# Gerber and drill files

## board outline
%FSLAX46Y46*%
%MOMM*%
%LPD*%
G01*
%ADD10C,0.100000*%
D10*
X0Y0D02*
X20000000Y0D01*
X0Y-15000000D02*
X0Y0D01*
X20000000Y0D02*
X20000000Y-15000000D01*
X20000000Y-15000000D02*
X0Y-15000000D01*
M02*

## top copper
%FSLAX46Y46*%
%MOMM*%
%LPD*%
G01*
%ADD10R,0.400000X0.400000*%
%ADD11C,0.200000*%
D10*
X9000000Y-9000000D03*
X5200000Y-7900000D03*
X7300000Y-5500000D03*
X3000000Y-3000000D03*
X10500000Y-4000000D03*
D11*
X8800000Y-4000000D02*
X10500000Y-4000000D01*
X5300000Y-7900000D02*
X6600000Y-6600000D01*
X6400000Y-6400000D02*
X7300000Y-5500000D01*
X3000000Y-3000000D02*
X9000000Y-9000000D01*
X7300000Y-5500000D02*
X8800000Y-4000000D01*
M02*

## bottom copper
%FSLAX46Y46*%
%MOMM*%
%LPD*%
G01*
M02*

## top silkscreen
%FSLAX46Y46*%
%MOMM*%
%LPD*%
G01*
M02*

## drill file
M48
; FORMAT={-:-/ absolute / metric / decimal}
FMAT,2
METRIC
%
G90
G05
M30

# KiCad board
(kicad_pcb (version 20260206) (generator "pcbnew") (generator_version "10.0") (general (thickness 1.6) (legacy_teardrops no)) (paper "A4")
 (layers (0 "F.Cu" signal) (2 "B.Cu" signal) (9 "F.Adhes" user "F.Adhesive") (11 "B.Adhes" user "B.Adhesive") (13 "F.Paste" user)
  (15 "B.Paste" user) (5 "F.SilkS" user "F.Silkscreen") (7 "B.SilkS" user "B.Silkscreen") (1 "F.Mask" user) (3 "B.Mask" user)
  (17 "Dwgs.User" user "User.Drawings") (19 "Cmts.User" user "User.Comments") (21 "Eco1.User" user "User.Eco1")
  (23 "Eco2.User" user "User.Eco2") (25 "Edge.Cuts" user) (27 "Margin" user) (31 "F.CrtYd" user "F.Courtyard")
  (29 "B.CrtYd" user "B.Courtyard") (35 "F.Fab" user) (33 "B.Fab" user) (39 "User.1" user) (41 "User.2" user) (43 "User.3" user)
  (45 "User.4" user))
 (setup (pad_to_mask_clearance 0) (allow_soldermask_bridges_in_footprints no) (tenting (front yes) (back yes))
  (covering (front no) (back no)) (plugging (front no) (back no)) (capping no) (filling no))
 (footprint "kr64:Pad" (layer "F.Cu") (at 9 9)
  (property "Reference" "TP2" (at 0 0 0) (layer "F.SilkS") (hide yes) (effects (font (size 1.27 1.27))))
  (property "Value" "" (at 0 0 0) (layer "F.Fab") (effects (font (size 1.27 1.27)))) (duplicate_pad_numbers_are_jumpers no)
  (pad "1" smd rect (at 0 0) (size 0.4 0.4) (layers "F.Cu" "F.Mask" "F.Paste") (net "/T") (thermal_bridge_angle 45)))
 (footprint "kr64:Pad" (layer "F.Cu") (at 5.2 7.9)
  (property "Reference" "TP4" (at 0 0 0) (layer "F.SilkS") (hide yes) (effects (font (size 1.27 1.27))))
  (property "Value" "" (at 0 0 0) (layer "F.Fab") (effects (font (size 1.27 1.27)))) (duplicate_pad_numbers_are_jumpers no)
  (pad "1" smd rect (at 0 0) (size 0.4 0.4) (layers "F.Cu" "F.Mask" "F.Paste") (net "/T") (thermal_bridge_angle 45)))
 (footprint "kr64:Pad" (layer "F.Cu") (at 7.3 5.5)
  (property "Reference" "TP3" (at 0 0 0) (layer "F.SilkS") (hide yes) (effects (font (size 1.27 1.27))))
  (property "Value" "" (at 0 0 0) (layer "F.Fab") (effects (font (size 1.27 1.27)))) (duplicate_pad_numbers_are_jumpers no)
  (pad "1" smd rect (at 0 0) (size 0.4 0.4) (layers "F.Cu" "F.Mask" "F.Paste") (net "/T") (thermal_bridge_angle 45)))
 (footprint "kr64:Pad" (layer "F.Cu") (at 3 3)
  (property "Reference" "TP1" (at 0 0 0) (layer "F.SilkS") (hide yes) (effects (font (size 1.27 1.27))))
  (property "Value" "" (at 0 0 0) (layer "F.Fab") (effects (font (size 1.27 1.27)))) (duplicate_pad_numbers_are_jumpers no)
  (pad "1" smd rect (at 0 0) (size 0.4 0.4) (layers "F.Cu" "F.Mask" "F.Paste") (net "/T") (thermal_bridge_angle 45)))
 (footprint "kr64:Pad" (layer "F.Cu") (at 10.5 4)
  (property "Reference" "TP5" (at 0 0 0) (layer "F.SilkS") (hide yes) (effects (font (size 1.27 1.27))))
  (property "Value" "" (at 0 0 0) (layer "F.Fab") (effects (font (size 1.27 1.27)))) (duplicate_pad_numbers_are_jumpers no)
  (pad "1" smd rect (at 0 0) (size 0.4 0.4) (layers "F.Cu" "F.Mask" "F.Paste") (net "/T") (thermal_bridge_angle 45)))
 (gr_line (start 0 0) (end 20 0) (stroke (width 0.1) (type default)) (layer "Edge.Cuts"))
 (gr_line (start 0 15) (end 0 0) (stroke (width 0.1) (type default)) (layer "Edge.Cuts"))
 (gr_line (start 20 0) (end 20 15) (stroke (width 0.1) (type default)) (layer "Edge.Cuts"))
 (gr_line (start 20 15) (end 0 15) (stroke (width 0.1) (type default)) (layer "Edge.Cuts"))
 (segment (start 8.8 4) (end 10.5 4) (width 0.2) (layer "F.Cu") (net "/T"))
 (segment (start 5.3 7.9) (end 6.6 6.6) (width 0.2) (layer "F.Cu") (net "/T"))
 (segment (start 6.4 6.4) (end 7.3 5.5) (width 0.2) (layer "F.Cu") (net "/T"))
 (segment (start 3 3) (end 9 9) (width 0.2) (layer "F.Cu") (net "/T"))
 (segment (start 7.3 5.5) (end 8.8 4) (width 0.2) (layer "F.Cu") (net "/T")))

